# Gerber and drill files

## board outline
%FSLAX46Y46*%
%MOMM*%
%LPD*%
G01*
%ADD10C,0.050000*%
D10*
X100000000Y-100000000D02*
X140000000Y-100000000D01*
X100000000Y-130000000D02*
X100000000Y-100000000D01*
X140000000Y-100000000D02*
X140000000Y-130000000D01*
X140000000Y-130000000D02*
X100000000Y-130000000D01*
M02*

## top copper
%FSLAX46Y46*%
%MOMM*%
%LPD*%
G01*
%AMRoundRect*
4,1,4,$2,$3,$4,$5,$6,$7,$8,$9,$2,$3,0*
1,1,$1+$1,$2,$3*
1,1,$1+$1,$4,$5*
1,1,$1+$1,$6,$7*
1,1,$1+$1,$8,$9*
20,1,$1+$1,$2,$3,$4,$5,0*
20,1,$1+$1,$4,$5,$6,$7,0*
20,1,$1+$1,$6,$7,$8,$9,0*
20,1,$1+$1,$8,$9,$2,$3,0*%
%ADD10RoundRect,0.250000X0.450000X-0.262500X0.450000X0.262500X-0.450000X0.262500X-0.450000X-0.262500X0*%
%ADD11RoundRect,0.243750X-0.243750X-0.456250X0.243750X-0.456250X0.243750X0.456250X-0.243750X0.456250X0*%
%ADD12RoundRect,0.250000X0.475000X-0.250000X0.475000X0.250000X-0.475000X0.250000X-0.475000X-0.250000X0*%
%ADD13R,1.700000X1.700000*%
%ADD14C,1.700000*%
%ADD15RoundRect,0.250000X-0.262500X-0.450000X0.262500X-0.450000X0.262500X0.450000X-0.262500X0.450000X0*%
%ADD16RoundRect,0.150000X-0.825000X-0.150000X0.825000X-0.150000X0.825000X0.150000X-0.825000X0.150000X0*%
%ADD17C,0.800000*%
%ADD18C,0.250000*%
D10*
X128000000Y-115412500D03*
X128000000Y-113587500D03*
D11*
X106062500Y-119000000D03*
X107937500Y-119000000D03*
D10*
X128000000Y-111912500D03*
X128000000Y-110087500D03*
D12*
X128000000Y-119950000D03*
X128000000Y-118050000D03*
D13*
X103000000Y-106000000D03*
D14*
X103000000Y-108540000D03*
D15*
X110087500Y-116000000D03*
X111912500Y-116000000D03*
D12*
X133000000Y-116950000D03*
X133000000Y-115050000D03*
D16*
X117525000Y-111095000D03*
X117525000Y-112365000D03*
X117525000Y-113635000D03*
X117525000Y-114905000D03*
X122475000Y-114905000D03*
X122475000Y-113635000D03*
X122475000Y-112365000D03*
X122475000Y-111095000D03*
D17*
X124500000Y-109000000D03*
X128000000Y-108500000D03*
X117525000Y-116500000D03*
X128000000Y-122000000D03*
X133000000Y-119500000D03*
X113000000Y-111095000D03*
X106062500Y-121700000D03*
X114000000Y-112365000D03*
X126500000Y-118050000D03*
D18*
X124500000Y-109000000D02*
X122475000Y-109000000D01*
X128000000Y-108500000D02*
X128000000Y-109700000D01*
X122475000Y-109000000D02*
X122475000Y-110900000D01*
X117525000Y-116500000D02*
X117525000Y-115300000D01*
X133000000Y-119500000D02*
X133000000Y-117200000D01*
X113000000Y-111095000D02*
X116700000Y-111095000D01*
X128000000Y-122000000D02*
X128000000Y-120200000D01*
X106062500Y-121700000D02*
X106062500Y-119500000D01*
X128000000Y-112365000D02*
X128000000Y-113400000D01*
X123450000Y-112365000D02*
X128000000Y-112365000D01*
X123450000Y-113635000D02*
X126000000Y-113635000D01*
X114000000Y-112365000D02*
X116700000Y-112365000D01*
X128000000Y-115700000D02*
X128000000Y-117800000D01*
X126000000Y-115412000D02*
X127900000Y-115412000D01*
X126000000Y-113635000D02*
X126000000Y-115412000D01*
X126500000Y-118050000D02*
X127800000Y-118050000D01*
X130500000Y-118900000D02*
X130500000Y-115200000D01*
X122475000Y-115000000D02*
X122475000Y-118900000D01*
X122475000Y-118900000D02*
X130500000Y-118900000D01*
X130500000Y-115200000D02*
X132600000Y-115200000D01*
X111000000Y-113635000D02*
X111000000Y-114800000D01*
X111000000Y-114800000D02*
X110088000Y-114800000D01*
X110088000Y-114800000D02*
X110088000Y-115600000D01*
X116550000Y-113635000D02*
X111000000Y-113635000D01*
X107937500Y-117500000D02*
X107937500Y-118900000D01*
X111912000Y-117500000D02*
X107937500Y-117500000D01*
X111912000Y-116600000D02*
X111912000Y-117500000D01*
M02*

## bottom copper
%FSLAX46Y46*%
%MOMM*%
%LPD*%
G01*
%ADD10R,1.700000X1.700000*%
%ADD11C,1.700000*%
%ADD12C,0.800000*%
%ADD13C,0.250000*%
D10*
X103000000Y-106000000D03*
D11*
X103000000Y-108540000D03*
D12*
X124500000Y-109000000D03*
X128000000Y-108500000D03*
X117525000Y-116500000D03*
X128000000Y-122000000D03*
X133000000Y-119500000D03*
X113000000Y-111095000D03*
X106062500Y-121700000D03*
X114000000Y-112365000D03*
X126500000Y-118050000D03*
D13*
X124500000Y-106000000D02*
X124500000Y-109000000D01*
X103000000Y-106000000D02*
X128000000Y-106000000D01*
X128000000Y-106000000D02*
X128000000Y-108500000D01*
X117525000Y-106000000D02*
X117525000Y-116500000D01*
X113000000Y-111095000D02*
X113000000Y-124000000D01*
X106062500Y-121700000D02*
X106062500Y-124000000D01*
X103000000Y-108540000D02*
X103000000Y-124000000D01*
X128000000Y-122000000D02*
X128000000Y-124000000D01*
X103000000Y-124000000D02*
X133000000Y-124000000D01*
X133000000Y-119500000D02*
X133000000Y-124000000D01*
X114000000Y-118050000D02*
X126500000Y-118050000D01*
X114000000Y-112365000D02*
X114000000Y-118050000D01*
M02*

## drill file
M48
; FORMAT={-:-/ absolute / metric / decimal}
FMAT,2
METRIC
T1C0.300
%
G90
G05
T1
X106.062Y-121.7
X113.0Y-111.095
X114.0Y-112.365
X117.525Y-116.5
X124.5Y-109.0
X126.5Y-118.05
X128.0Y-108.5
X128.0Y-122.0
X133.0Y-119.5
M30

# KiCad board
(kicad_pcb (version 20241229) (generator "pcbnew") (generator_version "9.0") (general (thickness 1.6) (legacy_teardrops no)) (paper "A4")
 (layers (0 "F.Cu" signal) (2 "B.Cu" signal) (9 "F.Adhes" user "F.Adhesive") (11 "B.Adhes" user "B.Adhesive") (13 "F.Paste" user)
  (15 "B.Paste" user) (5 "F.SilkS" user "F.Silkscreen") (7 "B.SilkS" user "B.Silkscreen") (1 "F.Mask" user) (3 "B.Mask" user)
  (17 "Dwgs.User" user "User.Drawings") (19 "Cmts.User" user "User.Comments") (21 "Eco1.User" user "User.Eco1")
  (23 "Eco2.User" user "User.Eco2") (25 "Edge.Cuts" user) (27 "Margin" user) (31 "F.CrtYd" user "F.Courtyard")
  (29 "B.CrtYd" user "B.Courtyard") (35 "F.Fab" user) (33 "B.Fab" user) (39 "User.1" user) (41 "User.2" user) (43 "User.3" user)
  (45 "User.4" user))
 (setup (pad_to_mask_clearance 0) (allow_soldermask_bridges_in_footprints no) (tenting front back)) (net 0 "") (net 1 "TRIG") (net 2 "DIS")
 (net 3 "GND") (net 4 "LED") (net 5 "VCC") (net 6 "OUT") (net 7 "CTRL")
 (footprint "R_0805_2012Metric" (layer "F.Cu") (at 128 114.5 90)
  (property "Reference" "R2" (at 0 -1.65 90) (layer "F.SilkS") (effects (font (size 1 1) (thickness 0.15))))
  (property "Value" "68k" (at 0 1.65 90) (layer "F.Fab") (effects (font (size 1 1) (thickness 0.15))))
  (pad "1" smd roundrect (at -0.9125 0 90) (size 1.025 1.4) (layers "F.Cu" "F.Mask" "F.Paste") (roundrect_rratio 0.243902) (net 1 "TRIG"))
  (pad "2" smd roundrect (at 0.9125 0 90) (size 1.025 1.4) (layers "F.Cu" "F.Mask" "F.Paste") (roundrect_rratio 0.243902) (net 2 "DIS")))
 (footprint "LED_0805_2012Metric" (layer "F.Cu") (at 107 119)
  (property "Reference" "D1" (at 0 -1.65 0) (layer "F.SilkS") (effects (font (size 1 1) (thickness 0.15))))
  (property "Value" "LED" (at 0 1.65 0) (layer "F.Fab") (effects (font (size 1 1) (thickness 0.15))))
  (pad "1" smd roundrect (at -0.9375 0) (size 0.975 1.4) (layers "F.Cu" "F.Mask" "F.Paste") (roundrect_rratio 0.25) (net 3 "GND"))
  (pad "2" smd roundrect (at 0.9375 0) (size 0.975 1.4) (layers "F.Cu" "F.Mask" "F.Paste") (roundrect_rratio 0.25) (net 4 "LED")))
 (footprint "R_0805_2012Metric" (layer "F.Cu") (at 128 111 90)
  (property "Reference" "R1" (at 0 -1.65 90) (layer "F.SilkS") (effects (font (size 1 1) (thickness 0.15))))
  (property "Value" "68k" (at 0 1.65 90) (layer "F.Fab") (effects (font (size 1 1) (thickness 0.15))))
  (pad "1" smd roundrect (at -0.9125 0 90) (size 1.025 1.4) (layers "F.Cu" "F.Mask" "F.Paste") (roundrect_rratio 0.243902) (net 2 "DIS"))
  (pad "2" smd roundrect (at 0.9125 0 90) (size 1.025 1.4) (layers "F.Cu" "F.Mask" "F.Paste") (roundrect_rratio 0.243902) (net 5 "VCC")))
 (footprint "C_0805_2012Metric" (layer "F.Cu") (at 128 119 90)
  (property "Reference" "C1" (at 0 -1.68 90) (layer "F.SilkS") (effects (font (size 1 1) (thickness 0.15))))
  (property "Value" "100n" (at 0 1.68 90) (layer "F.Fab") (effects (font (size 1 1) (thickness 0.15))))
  (pad "1" smd roundrect (at -0.95 0 90) (size 1 1.45) (layers "F.Cu" "F.Mask" "F.Paste") (roundrect_rratio 0.25) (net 3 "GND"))
  (pad "2" smd roundrect (at 0.95 0 90) (size 1 1.45) (layers "F.Cu" "F.Mask" "F.Paste") (roundrect_rratio 0.25) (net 1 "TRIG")))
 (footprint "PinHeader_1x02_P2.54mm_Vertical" (layer "F.Cu") (at 103 106)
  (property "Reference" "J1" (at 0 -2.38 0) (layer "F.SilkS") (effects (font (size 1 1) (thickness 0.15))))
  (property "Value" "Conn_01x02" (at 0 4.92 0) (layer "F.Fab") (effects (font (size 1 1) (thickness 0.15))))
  (pad "1" thru_hole rect (at 0 0) (size 1.7 1.7) (drill 0) (layers "*.Cu" "*.Mask") (remove_unused_layers no) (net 5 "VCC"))
  (pad "2" thru_hole circle (at 0 2.54) (size 1.7 1.7) (drill 0) (layers "*.Cu" "*.Mask") (remove_unused_layers no) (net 3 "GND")))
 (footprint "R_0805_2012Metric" (layer "F.Cu") (at 111 116)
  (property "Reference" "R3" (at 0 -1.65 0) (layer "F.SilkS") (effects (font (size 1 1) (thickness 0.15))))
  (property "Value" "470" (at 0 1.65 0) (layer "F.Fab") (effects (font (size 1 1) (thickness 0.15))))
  (pad "1" smd roundrect (at -0.9125 0) (size 1.025 1.4) (layers "F.Cu" "F.Mask" "F.Paste") (roundrect_rratio 0.243902) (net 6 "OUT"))
  (pad "2" smd roundrect (at 0.9125 0) (size 1.025 1.4) (layers "F.Cu" "F.Mask" "F.Paste") (roundrect_rratio 0.243902) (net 4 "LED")))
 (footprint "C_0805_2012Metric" (layer "F.Cu") (at 133 116 90)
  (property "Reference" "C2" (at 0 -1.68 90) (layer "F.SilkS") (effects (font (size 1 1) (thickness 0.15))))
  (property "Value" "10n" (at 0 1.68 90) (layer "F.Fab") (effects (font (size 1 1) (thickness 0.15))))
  (pad "1" smd roundrect (at -0.95 0 90) (size 1 1.45) (layers "F.Cu" "F.Mask" "F.Paste") (roundrect_rratio 0.25) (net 3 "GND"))
  (pad "2" smd roundrect (at 0.95 0 90) (size 1 1.45) (layers "F.Cu" "F.Mask" "F.Paste") (roundrect_rratio 0.25) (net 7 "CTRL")))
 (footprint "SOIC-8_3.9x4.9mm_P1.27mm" (layer "F.Cu") (at 120 113)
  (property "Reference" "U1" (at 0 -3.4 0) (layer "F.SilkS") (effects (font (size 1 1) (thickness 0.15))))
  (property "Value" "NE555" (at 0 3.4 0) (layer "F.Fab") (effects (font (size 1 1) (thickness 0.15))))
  (pad "1" smd roundrect (at -2.475 -1.905) (size 1.95 0.6) (layers "F.Cu" "F.Mask" "F.Paste") (roundrect_rratio 0.25) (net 3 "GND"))
  (pad "2" smd roundrect (at -2.475 -0.635) (size 1.95 0.6) (layers "F.Cu" "F.Mask" "F.Paste") (roundrect_rratio 0.25) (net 1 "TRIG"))
  (pad "3" smd roundrect (at -2.475 0.635) (size 1.95 0.6) (layers "F.Cu" "F.Mask" "F.Paste") (roundrect_rratio 0.25) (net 6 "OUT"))
  (pad "4" smd roundrect (at -2.475 1.905) (size 1.95 0.6) (layers "F.Cu" "F.Mask" "F.Paste") (roundrect_rratio 0.25) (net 5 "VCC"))
  (pad "5" smd roundrect (at 2.475 1.905) (size 1.95 0.6) (layers "F.Cu" "F.Mask" "F.Paste") (roundrect_rratio 0.25) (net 7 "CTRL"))
  (pad "6" smd roundrect (at 2.475 0.635) (size 1.95 0.6) (layers "F.Cu" "F.Mask" "F.Paste") (roundrect_rratio 0.25) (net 1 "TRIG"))
  (pad "7" smd roundrect (at 2.475 -0.635) (size 1.95 0.6) (layers "F.Cu" "F.Mask" "F.Paste") (roundrect_rratio 0.25) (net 2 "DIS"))
  (pad "8" smd roundrect (at 2.475 -1.905) (size 1.95 0.6) (layers "F.Cu" "F.Mask" "F.Paste") (roundrect_rratio 0.25) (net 5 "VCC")))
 (gr_line (start 100 100) (end 140 100) (stroke (width 0.05) (type default)) (layer "Edge.Cuts"))
 (gr_line (start 100 130) (end 100 100) (stroke (width 0.05) (type default)) (layer "Edge.Cuts"))
 (gr_line (start 140 100) (end 140 130) (stroke (width 0.05) (type default)) (layer "Edge.Cuts"))
 (gr_line (start 140 130) (end 100 130) (stroke (width 0.05) (type default)) (layer "Edge.Cuts"))
 (segment (start 124.5 109) (end 122.475 109) (width 0.25) (layer "F.Cu") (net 5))
 (segment (start 128 108.5) (end 128 109.7) (width 0.25) (layer "F.Cu") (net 5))
 (segment (start 122.475 109) (end 122.475 110.9) (width 0.25) (layer "F.Cu") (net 5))
 (segment (start 117.525 116.5) (end 117.525 115.3) (width 0.25) (layer "F.Cu") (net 5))
 (via (at 124.5 109) (size 0.8) (drill 0) (layers "F.Cu" "B.Cu") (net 5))
 (via (at 128 108.5) (size 0.8) (drill 0) (layers "F.Cu" "B.Cu") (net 5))
 (via (at 117.525 116.5) (size 0.8) (drill 0) (layers "F.Cu" "B.Cu") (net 5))
 (segment (start 124.5 106) (end 124.5 109) (width 0.25) (layer "B.Cu") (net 5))
 (segment (start 103 106) (end 128 106) (width 0.25) (layer "B.Cu") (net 5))
 (segment (start 128 106) (end 128 108.5) (width 0.25) (layer "B.Cu") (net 5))
 (segment (start 117.525 106) (end 117.525 116.5) (width 0.25) (layer "B.Cu") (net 5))
 (segment (start 133 119.5) (end 133 117.2) (width 0.25) (layer "F.Cu") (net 3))
 (segment (start 113 111.095) (end 116.7 111.095) (width 0.25) (layer "F.Cu") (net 3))
 (segment (start 128 122) (end 128 120.2) (width 0.25) (layer "F.Cu") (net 3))
 (segment (start 106.0625 121.7) (end 106.0625 119.5) (width 0.25) (layer "F.Cu") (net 3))
 (via (at 128 122) (size 0.8) (drill 0) (layers "F.Cu" "B.Cu") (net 3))
 (via (at 133 119.5) (size 0.8) (drill 0) (layers "F.Cu" "B.Cu") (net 3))
 (via (at 113 111.095) (size 0.8) (drill 0) (layers "F.Cu" "B.Cu") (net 3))
 (via (at 106.0625 121.7) (size 0.8) (drill 0) (layers "F.Cu" "B.Cu") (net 3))
 (segment (start 113 111.095) (end 113 124) (width 0.25) (layer "B.Cu") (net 3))
 (segment (start 106.0625 121.7) (end 106.0625 124) (width 0.25) (layer "B.Cu") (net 3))
 (segment (start 103 108.54) (end 103 124) (width 0.25) (layer "B.Cu") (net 3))
 (segment (start 128 122) (end 128 124) (width 0.25) (layer "B.Cu") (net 3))
 (segment (start 103 124) (end 133 124) (width 0.25) (layer "B.Cu") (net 3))
 (segment (start 133 119.5) (end 133 124) (width 0.25) (layer "B.Cu") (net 3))
 (segment (start 128 112.365) (end 128 113.4) (width 0.25) (layer "F.Cu") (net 2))
 (segment (start 123.45 112.365) (end 128 112.365) (width 0.25) (layer "F.Cu") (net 2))
 (segment (start 123.45 113.635) (end 126 113.635) (width 0.25) (layer "F.Cu") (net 1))
 (segment (start 114 112.365) (end 116.7 112.365) (width 0.25) (layer "F.Cu") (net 1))
 (segment (start 128 115.7) (end 128 117.8) (width 0.25) (layer "F.Cu") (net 1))
 (segment (start 126 115.412) (end 127.9 115.412) (width 0.25) (layer "F.Cu") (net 1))
 (segment (start 126 113.635) (end 126 115.412) (width 0.25) (layer "F.Cu") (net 1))
 (segment (start 126.5 118.05) (end 127.8 118.05) (width 0.25) (layer "F.Cu") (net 1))
 (via (at 114 112.365) (size 0.8) (drill 0) (layers "F.Cu" "B.Cu") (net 1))
 (via (at 126.5 118.05) (size 0.8) (drill 0) (layers "F.Cu" "B.Cu") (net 1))
 (segment (start 114 118.05) (end 126.5 118.05) (width 0.25) (layer "B.Cu") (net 1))
 (segment (start 114 112.365) (end 114 118.05) (width 0.25) (layer "B.Cu") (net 1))
 (segment (start 130.5 118.9) (end 130.5 115.2) (width 0.25) (layer "F.Cu") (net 7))
 (segment (start 122.475 115) (end 122.475 118.9) (width 0.25) (layer "F.Cu") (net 7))
 (segment (start 122.475 118.9) (end 130.5 118.9) (width 0.25) (layer "F.Cu") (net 7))
 (segment (start 130.5 115.2) (end 132.6 115.2) (width 0.25) (layer "F.Cu") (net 7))
 (segment (start 111 113.635) (end 111 114.8) (width 0.25) (layer "F.Cu") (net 6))
 (segment (start 111 114.8) (end 110.088 114.8) (width 0.25) (layer "F.Cu") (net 6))
 (segment (start 110.088 114.8) (end 110.088 115.6) (width 0.25) (layer "F.Cu") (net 6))
 (segment (start 116.55 113.635) (end 111 113.635) (width 0.25) (layer "F.Cu") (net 6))
 (segment (start 107.9375 117.5) (end 107.9375 118.9) (width 0.25) (layer "F.Cu") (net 4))
 (segment (start 111.912 117.5) (end 107.9375 117.5) (width 0.25) (layer "F.Cu") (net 4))
 (segment (start 111.912 116.6) (end 111.912 117.5) (width 0.25) (layer "F.Cu") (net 4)))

